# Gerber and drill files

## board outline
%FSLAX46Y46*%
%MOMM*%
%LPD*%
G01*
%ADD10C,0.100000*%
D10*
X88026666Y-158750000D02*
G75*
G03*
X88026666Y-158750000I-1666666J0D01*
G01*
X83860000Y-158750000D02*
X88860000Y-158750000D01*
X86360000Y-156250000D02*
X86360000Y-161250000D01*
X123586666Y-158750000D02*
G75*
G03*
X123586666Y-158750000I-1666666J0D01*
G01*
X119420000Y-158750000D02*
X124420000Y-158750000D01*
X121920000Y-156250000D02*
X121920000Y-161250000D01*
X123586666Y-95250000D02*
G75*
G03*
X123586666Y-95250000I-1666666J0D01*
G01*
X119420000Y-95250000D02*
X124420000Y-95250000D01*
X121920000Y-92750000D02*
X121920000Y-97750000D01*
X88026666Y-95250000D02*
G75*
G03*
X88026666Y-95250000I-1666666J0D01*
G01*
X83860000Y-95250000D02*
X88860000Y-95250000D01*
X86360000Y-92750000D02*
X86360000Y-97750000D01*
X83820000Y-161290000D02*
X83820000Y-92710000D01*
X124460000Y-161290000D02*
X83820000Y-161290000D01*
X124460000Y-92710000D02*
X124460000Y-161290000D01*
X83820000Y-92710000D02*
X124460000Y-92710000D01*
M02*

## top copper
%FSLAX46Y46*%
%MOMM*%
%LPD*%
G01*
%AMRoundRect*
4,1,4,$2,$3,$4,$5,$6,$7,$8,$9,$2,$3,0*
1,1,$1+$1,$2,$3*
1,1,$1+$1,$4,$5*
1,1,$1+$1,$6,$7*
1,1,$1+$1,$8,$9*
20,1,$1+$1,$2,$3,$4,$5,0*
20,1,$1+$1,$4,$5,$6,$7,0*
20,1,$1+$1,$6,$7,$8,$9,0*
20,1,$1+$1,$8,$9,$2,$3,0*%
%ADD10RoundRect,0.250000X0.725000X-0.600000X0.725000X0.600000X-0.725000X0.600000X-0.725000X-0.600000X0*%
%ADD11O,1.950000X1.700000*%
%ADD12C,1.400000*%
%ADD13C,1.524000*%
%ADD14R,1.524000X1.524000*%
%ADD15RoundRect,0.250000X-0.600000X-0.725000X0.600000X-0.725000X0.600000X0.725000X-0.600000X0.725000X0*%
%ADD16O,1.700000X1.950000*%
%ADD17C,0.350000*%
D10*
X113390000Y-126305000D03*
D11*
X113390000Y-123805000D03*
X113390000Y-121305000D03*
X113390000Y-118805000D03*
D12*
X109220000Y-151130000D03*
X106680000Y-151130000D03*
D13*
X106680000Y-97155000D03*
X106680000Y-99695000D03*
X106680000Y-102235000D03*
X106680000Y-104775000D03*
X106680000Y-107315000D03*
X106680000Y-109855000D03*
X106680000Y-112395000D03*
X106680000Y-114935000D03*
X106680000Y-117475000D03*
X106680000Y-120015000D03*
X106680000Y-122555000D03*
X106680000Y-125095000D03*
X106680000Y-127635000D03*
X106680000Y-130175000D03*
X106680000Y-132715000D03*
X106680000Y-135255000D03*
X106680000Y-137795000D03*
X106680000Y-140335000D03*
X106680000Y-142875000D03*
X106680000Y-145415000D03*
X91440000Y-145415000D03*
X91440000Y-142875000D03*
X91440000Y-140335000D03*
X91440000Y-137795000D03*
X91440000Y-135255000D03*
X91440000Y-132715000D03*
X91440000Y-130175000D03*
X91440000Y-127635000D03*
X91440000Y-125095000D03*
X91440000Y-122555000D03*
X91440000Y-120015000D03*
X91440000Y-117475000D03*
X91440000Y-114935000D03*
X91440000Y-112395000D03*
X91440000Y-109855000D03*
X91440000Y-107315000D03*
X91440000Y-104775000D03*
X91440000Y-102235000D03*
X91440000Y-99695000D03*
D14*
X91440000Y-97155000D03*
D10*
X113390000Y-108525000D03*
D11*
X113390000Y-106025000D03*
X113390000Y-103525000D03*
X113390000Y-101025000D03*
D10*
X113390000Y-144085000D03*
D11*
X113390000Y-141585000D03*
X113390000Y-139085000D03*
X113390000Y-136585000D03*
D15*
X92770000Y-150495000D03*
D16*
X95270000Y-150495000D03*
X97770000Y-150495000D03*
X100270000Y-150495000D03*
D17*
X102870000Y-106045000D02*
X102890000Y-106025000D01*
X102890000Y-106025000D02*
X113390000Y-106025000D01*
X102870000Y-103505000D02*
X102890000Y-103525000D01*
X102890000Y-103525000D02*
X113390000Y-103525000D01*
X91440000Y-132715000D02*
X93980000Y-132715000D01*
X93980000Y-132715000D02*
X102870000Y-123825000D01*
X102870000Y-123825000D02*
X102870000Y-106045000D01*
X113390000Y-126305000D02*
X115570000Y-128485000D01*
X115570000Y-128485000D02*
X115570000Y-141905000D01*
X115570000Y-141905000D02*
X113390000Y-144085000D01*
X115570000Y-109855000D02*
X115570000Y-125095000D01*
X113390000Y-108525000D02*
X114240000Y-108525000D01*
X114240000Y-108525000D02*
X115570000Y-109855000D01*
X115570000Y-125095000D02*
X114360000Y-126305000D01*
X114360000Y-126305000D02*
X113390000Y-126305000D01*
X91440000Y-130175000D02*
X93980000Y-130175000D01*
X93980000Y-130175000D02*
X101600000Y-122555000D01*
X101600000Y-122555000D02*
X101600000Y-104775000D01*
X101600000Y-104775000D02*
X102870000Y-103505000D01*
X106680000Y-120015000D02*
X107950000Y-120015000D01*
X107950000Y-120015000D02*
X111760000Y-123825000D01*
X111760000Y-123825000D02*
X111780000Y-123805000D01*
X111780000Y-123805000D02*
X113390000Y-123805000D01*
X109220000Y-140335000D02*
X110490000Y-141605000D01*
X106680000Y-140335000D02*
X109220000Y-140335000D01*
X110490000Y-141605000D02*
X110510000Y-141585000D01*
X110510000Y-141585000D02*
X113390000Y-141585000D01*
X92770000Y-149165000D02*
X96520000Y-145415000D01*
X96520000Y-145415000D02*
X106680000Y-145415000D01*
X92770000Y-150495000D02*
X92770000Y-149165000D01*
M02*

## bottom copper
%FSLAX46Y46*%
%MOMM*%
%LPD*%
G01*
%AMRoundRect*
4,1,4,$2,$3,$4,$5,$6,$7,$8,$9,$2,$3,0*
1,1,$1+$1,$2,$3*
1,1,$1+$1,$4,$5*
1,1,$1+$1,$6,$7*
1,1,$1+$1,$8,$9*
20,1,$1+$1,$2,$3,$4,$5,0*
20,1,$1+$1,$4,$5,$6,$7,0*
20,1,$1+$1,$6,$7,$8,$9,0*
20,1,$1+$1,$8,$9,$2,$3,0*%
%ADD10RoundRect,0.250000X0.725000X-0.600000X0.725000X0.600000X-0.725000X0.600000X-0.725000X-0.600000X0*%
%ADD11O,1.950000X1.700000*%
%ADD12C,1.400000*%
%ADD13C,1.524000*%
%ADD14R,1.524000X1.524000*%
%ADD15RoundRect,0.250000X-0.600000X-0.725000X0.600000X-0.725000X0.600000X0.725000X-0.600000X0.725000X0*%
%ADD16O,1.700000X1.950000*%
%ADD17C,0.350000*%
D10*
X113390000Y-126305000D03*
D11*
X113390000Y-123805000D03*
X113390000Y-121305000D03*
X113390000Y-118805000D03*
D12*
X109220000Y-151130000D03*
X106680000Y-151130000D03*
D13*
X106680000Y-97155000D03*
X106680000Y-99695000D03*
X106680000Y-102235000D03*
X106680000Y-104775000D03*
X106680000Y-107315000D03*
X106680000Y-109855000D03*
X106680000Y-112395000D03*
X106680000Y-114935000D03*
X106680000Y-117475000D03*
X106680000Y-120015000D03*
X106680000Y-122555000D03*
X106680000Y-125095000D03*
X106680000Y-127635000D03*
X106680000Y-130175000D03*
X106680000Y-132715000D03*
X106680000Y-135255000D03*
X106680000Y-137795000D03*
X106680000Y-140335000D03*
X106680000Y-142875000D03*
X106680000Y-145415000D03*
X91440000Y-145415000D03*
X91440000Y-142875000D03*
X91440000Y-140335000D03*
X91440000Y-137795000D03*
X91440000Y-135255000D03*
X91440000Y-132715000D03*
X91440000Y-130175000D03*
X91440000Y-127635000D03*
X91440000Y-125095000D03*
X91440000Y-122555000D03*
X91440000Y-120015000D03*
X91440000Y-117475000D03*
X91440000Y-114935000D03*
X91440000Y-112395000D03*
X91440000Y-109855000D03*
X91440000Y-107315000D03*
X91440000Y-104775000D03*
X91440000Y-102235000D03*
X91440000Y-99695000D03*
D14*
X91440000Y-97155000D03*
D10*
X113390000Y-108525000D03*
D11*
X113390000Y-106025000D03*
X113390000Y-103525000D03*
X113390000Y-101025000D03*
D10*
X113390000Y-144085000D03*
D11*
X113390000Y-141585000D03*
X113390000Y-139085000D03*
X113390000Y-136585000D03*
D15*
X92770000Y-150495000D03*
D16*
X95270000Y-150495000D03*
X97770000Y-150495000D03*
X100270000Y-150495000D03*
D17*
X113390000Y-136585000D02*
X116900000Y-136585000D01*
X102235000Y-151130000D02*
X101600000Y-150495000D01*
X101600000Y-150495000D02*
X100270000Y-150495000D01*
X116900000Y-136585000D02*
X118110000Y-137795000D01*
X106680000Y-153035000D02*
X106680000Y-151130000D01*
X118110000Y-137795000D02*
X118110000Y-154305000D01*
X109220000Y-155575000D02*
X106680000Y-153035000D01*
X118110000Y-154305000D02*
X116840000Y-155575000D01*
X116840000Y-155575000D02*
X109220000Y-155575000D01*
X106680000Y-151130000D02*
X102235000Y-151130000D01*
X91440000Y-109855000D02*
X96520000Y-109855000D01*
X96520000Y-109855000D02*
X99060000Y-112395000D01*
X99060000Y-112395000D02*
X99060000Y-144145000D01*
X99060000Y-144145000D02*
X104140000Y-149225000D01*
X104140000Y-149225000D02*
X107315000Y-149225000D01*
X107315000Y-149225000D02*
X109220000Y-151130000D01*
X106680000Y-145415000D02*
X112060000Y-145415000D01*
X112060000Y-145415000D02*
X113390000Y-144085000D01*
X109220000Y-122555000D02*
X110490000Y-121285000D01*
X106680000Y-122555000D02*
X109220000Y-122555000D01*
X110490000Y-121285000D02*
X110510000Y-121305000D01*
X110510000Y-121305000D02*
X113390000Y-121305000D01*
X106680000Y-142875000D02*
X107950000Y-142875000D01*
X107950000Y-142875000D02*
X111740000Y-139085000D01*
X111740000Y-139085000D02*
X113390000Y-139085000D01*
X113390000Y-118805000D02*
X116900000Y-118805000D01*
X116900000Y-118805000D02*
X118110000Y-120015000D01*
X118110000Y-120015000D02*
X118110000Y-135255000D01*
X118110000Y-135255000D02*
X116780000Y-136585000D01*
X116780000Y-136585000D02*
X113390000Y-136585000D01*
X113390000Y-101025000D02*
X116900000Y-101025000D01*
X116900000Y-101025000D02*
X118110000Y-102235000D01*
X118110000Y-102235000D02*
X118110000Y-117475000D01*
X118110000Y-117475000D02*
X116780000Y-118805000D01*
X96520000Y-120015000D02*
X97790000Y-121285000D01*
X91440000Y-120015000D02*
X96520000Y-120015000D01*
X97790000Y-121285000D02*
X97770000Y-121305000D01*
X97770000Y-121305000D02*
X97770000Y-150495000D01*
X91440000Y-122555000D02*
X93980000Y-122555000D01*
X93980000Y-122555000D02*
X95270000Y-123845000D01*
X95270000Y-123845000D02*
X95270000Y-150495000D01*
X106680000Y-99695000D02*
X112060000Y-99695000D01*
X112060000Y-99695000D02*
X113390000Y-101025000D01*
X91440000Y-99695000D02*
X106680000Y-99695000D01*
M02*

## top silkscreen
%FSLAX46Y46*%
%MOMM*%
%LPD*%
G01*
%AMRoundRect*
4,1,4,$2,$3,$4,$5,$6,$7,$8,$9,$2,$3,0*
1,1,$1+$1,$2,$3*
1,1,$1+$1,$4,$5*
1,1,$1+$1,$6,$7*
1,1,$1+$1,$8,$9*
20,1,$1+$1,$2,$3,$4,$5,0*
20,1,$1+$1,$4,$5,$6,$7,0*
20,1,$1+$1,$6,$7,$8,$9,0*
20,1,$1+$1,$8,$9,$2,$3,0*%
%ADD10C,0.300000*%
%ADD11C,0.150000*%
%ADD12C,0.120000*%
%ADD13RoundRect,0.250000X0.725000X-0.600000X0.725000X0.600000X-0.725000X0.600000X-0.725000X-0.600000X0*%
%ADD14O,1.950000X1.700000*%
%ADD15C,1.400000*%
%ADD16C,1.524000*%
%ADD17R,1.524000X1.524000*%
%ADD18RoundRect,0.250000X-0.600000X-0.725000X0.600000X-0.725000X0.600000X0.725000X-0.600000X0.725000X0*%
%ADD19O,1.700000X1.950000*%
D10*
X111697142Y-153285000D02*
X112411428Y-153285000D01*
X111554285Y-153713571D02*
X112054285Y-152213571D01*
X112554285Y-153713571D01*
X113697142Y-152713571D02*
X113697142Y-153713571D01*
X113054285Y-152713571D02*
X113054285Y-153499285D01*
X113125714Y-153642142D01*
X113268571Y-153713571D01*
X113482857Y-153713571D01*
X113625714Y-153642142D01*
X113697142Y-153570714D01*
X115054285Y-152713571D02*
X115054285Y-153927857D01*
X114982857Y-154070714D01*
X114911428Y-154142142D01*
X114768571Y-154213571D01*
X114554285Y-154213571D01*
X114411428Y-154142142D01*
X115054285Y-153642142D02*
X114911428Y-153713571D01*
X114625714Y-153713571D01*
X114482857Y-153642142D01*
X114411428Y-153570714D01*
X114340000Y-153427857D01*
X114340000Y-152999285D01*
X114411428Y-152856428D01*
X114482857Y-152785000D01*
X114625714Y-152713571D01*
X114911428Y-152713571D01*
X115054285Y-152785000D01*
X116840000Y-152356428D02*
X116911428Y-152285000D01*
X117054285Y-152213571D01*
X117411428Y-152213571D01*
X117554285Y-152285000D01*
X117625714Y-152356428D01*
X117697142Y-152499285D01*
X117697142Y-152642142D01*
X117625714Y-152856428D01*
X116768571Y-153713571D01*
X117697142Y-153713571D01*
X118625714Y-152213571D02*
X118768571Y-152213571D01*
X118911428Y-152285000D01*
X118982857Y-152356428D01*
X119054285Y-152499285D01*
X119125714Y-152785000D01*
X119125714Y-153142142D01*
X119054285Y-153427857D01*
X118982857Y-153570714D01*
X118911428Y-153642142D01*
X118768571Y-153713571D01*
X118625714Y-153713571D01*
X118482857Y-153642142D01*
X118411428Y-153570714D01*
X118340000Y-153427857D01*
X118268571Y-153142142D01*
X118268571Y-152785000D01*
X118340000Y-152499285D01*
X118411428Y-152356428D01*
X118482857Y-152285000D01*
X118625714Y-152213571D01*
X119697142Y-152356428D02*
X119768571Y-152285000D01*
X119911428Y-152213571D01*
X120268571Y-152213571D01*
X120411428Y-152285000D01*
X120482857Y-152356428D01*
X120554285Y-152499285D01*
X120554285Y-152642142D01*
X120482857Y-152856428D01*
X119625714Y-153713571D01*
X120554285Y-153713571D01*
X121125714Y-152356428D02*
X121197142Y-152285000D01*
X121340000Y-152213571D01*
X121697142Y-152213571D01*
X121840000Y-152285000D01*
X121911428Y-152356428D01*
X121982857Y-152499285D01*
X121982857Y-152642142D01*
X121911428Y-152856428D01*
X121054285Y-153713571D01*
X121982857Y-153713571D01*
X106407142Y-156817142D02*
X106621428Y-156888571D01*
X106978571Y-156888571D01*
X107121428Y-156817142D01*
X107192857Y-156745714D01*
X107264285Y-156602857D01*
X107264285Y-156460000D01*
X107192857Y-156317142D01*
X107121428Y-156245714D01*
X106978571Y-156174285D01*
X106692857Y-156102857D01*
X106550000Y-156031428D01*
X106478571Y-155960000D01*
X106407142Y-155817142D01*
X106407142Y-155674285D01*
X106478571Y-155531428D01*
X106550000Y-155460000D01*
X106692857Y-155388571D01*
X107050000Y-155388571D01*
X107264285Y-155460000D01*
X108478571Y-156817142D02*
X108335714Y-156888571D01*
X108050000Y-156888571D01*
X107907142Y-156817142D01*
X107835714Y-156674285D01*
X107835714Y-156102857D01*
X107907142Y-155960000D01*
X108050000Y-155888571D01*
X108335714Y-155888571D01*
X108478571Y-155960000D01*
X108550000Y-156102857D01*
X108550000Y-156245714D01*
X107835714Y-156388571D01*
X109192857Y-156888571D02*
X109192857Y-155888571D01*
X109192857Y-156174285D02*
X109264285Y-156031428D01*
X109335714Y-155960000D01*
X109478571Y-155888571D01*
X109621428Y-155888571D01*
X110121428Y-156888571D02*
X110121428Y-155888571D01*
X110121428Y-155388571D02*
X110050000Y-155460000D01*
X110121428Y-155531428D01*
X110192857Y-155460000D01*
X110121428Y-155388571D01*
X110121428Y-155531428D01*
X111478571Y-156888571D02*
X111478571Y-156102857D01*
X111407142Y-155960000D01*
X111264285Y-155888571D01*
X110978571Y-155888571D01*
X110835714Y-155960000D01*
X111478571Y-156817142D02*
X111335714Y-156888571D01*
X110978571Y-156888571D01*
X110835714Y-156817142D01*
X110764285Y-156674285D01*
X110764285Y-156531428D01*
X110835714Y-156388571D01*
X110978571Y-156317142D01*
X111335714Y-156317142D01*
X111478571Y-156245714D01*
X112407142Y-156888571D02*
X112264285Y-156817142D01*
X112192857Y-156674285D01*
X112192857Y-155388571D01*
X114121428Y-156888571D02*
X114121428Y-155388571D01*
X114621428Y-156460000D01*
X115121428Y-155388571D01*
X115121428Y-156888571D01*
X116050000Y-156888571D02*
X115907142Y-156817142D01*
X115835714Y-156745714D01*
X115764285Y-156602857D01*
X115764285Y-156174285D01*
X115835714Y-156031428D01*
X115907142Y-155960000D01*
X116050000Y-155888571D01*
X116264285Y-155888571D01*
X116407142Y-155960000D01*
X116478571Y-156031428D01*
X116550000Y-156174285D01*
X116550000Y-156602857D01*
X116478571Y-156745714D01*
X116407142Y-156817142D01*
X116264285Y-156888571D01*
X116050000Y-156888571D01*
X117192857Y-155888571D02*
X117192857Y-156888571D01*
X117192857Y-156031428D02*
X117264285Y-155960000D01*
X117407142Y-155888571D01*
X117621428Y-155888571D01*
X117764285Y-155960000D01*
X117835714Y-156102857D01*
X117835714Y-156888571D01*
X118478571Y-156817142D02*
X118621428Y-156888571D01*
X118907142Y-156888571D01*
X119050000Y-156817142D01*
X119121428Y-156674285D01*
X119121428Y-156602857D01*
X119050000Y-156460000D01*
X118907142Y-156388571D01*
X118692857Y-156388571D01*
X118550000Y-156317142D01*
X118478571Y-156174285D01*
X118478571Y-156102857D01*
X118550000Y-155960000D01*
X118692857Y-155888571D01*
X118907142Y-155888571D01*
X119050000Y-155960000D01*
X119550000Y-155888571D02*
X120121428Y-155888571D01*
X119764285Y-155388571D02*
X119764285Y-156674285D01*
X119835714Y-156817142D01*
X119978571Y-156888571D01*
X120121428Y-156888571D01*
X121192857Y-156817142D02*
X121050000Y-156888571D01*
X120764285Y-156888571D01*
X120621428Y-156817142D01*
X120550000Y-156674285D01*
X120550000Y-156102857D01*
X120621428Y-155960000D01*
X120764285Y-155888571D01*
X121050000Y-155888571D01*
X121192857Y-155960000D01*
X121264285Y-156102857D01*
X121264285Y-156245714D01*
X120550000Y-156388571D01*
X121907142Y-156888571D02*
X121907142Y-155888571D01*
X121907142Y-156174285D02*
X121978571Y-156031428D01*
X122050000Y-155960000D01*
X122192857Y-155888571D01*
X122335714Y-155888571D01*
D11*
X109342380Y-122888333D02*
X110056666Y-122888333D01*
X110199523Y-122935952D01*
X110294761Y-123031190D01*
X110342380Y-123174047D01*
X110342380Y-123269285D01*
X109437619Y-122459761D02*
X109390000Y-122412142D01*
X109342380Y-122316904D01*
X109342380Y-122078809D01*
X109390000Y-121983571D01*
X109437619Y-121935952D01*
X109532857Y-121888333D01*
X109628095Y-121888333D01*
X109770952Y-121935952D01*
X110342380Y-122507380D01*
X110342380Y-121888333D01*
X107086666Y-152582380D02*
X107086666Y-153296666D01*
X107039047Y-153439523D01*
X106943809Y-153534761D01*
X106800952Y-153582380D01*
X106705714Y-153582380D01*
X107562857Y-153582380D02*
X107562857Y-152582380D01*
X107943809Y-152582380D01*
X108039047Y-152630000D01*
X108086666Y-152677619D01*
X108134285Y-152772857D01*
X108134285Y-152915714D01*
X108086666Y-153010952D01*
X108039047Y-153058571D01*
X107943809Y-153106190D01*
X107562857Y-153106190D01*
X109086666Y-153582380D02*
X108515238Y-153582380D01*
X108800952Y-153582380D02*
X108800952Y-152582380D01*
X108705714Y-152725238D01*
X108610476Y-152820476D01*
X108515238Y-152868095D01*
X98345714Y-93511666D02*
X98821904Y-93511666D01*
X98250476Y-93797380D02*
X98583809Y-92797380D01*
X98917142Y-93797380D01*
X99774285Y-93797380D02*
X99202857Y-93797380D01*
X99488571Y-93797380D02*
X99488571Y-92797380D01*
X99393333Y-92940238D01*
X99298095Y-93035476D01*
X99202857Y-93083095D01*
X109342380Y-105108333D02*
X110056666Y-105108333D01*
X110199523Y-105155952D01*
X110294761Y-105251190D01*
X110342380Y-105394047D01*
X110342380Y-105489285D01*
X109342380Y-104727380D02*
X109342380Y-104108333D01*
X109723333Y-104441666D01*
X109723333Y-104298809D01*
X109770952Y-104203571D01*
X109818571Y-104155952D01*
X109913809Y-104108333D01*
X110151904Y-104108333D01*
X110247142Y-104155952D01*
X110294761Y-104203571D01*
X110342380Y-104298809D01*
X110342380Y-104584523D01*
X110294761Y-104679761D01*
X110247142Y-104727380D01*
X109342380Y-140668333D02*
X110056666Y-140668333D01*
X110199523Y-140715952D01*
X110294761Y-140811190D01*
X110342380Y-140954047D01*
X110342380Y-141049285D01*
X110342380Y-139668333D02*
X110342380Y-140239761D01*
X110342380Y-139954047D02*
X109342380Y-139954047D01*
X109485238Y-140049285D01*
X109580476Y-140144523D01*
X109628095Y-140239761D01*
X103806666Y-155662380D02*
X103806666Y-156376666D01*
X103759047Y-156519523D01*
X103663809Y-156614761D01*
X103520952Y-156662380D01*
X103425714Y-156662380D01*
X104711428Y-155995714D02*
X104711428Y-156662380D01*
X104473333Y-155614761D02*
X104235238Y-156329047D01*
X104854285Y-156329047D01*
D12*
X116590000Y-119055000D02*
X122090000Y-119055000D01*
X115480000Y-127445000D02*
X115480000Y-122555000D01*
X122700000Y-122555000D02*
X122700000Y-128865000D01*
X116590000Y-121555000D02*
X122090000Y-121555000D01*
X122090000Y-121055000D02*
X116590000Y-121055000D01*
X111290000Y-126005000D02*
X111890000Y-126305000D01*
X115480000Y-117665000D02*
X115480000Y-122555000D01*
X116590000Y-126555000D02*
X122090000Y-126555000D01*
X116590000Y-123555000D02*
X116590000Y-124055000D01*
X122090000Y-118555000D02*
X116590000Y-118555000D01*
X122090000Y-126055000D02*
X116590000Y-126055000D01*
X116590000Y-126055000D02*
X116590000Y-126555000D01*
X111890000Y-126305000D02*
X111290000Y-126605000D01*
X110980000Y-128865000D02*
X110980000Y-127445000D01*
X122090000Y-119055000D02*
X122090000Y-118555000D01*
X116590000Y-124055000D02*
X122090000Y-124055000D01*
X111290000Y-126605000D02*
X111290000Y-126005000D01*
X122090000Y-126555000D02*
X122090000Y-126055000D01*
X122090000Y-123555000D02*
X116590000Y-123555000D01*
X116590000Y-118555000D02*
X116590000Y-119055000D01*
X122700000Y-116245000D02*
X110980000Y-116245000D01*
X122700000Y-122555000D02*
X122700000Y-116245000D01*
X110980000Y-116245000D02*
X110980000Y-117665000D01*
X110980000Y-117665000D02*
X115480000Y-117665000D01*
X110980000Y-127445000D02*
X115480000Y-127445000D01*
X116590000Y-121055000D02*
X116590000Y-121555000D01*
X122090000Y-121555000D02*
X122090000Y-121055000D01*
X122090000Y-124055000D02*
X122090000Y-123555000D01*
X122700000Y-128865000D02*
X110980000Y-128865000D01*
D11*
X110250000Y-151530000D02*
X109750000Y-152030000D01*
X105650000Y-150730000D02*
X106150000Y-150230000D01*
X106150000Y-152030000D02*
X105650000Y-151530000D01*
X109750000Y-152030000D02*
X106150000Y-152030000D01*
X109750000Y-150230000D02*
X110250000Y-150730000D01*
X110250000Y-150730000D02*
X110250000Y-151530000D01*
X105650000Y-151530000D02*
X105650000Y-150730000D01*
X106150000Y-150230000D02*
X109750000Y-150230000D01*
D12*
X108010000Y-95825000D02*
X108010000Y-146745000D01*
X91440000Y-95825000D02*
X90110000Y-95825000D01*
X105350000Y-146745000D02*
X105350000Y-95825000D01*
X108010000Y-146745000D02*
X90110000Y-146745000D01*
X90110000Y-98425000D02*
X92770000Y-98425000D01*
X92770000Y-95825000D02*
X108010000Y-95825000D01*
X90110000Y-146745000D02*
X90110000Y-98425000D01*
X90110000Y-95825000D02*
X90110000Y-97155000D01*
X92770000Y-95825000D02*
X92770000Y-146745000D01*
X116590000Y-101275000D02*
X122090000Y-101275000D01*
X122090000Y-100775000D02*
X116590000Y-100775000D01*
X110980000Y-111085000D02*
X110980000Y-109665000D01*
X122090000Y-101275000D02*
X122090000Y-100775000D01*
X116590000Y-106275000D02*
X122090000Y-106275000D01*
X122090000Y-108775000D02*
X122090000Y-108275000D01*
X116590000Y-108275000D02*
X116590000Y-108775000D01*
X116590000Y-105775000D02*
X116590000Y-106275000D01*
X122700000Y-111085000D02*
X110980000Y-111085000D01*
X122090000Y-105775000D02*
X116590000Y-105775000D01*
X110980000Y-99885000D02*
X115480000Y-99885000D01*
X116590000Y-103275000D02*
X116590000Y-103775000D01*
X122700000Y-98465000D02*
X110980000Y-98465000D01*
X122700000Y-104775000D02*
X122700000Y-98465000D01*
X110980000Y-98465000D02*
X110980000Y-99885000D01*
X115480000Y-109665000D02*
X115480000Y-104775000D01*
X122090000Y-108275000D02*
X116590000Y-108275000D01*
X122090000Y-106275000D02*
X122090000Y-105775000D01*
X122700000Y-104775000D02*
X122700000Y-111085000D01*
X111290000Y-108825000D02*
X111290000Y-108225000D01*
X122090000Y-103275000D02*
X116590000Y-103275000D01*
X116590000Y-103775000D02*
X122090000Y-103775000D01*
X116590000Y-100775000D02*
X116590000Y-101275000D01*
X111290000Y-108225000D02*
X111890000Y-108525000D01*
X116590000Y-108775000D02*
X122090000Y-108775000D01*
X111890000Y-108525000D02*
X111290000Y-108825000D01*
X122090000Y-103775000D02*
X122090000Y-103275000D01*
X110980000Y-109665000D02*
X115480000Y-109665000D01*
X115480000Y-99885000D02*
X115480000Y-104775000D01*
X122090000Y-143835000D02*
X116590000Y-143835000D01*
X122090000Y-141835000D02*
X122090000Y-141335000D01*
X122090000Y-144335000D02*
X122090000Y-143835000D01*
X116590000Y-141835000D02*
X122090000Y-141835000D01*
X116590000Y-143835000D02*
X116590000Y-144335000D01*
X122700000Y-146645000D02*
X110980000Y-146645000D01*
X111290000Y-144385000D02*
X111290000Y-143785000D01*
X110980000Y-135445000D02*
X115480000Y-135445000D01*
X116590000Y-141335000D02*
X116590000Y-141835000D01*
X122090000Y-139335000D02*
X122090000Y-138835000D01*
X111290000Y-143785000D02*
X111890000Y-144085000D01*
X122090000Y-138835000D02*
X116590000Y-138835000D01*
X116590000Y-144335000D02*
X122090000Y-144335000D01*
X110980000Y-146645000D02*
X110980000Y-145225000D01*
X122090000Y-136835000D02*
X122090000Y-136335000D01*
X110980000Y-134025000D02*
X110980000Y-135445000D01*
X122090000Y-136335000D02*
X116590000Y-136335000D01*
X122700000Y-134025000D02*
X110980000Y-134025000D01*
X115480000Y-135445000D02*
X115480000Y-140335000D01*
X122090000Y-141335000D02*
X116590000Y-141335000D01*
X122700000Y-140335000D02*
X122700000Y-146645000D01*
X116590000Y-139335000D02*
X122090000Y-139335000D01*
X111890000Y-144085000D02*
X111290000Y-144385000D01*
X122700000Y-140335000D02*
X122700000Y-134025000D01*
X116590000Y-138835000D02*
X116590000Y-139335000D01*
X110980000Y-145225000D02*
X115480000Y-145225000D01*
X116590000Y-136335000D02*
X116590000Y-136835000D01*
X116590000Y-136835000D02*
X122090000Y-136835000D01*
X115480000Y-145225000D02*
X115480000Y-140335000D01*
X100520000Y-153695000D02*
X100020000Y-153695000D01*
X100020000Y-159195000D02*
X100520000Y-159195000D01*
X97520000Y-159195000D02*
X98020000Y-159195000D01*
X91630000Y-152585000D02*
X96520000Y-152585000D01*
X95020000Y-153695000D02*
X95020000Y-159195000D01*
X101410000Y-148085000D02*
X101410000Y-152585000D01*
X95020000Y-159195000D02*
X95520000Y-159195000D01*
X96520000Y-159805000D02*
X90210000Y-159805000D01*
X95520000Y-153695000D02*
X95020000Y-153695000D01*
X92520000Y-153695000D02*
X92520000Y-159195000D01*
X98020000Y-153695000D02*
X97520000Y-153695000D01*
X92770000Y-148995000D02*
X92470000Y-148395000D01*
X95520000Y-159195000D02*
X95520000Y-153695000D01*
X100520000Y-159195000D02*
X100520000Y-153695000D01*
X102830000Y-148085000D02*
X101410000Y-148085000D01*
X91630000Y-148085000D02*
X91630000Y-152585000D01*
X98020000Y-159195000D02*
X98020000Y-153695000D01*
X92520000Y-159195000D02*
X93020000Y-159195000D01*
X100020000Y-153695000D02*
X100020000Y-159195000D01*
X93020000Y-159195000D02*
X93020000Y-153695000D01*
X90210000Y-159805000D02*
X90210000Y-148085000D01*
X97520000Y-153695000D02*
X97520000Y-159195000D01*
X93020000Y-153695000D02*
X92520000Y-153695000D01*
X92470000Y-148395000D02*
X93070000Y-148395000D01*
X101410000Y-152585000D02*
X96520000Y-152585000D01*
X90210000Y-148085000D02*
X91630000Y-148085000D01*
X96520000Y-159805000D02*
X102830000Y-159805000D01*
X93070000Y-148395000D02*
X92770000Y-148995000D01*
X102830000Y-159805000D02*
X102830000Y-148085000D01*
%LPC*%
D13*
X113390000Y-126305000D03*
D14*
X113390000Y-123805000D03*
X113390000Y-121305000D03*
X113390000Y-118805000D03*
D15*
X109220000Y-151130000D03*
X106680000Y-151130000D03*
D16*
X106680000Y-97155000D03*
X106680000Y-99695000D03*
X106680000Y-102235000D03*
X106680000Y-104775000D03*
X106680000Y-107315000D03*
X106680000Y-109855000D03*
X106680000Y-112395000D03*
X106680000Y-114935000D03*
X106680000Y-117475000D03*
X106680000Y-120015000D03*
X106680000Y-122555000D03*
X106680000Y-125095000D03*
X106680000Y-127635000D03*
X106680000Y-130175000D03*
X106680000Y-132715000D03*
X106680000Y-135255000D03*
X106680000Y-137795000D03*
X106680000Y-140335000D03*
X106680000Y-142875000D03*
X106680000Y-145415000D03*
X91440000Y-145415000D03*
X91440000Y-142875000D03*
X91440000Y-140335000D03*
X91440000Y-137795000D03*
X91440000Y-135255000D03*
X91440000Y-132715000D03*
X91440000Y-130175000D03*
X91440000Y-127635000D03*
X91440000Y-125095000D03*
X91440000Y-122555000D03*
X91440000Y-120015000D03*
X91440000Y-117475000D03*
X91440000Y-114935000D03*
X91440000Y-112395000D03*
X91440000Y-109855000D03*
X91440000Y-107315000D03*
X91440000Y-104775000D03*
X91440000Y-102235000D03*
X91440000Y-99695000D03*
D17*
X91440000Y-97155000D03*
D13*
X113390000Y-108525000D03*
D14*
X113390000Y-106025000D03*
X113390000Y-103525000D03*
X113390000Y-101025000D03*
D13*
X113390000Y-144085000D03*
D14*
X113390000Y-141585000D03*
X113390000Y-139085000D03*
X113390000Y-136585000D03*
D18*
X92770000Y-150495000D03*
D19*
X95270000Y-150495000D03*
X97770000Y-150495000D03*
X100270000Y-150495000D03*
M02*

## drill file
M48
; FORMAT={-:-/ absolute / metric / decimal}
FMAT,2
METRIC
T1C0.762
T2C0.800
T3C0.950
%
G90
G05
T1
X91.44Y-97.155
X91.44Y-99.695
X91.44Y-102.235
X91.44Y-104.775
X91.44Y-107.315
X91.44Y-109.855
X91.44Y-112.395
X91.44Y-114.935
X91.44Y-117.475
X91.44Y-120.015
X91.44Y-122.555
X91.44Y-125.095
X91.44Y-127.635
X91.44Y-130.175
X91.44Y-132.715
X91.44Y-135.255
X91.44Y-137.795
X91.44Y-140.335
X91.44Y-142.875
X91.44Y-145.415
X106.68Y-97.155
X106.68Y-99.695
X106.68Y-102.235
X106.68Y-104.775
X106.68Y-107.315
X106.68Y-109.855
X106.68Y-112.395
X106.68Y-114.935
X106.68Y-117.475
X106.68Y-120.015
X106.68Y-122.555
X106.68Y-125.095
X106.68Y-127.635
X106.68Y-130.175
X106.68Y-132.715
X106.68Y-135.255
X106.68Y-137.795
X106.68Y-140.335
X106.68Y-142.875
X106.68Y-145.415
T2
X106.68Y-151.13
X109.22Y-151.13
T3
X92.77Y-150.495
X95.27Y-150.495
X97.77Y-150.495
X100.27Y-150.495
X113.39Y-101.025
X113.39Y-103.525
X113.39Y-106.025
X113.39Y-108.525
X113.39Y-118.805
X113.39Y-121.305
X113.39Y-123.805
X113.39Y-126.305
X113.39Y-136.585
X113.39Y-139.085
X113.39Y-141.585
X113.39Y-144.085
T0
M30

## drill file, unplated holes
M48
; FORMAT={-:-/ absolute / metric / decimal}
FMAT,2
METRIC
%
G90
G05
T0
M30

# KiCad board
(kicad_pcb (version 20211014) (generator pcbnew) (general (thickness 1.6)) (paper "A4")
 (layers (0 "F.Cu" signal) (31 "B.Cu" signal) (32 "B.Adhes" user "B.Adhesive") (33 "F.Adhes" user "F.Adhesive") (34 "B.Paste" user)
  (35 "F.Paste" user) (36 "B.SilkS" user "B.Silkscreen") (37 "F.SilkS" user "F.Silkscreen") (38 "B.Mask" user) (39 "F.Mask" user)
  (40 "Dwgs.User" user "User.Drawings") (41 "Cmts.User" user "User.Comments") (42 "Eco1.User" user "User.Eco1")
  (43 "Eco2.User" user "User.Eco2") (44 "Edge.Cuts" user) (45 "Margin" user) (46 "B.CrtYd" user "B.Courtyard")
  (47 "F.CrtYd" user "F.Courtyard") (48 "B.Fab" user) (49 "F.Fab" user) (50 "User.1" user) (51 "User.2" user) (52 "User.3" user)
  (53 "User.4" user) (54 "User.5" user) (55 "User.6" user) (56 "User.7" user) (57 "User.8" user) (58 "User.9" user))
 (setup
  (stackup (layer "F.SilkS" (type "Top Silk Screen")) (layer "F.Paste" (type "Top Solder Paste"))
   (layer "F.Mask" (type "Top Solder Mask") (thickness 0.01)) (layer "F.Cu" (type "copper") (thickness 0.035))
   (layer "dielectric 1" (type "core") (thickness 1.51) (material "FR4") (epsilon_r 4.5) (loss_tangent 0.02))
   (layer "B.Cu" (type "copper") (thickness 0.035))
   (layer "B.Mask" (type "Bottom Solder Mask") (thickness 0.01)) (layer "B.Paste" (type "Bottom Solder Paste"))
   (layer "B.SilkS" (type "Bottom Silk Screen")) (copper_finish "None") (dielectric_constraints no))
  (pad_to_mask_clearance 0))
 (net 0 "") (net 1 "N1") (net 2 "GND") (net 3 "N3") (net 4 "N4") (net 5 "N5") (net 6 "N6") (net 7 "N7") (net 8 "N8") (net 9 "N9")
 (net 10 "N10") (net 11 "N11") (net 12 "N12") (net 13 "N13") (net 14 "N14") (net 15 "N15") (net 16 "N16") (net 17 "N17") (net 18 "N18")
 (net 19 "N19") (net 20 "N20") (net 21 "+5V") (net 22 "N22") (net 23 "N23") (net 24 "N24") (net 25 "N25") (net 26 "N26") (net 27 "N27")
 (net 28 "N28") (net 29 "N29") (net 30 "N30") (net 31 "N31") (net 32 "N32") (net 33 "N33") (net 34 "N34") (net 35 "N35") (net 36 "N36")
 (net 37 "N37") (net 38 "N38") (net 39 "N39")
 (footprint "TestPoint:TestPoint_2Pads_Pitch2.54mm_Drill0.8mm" (layer "F.Cu") (at 109.22 151.13 180)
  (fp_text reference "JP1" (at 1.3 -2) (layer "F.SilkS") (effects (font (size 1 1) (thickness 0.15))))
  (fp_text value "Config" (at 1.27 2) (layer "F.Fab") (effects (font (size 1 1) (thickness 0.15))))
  (fp_line (start -1.03 0.4) (end -1.03 -0.4) (layer "F.SilkS") (width 0.15))
  (fp_line (start -0.53 0.9) (end -1.03 0.4) (layer "F.SilkS") (width 0.15))
  (fp_line (start -1.03 -0.4) (end -0.53 -0.9) (layer "F.SilkS") (width 0.15))
  (fp_line (start 3.07 -0.9) (end 3.57 -0.4) (layer "F.SilkS") (width 0.15))
  (fp_line (start 3.07 0.9) (end -0.53 0.9) (layer "F.SilkS") (width 0.15))
  (fp_line (start 3.57 -0.4) (end 3.57 0.4) (layer "F.SilkS") (width 0.15))
  (fp_line (start 3.57 0.4) (end 3.07 0.9) (layer "F.SilkS") (width 0.15))
  (fp_line (start -0.53 -0.9) (end 3.07 -0.9) (layer "F.SilkS") (width 0.15))
  (pad "1" thru_hole circle (at 0 0 180) (size 1.4 1.4) (drill 0.8) (layers *.Cu *.Mask) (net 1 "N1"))
  (pad "2" thru_hole circle (at 2.54 0 180) (size 1.4 1.4) (drill 0.8) (layers *.Cu *.Mask) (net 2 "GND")))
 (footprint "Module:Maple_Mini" (layer "F.Cu") (at 91.44 97.155)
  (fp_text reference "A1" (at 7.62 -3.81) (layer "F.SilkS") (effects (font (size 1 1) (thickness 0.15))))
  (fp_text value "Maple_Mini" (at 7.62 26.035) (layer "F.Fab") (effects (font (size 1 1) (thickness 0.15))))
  (fp_line (start 1.33 -1.33) (end 1.33 49.59) (layer "F.SilkS") (width 0.12))
  (fp_line (start -1.33 -1.33) (end -1.33 0) (layer "F.SilkS") (width 0.12))
  (fp_line (start -1.33 49.59) (end -1.33 1.27) (layer "F.SilkS") (width 0.12))
  (fp_line (start 1.33 -1.33) (end 16.57 -1.33) (layer "F.SilkS") (width 0.12))
  (fp_line (start -1.33 1.27) (end 1.33 1.27) (layer "F.SilkS") (width 0.12))
  (fp_line (start 16.57 49.59) (end -1.33 49.59) (layer "F.SilkS") (width 0.12))
  (fp_line (start 13.91 49.59) (end 13.91 -1.33) (layer "F.SilkS") (width 0.12))
  (fp_line (start 0 -1.33) (end -1.33 -1.33) (layer "F.SilkS") (width 0.12))
  (fp_line (start 16.57 -1.33) (end 16.57 49.59) (layer "F.SilkS") (width 0.12))
  (pad "1" thru_hole rect (at 0 0) (size 1.524 1.524) (drill 0.762) (layers *.Cu *.Mask) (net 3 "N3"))
  (pad "2" thru_hole circle (at 0 2.54) (size 1.524 1.524) (drill 0.762) (layers *.Cu *.Mask) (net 2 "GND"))
  (pad "3" thru_hole circle (at 0 5.08) (size 1.524 1.524) (drill 0.762) (layers *.Cu *.Mask) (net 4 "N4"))
  (pad "4" thru_hole circle (at 0 7.62) (size 1.524 1.524) (drill 0.762) (layers *.Cu *.Mask) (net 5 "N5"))
  (pad "5" thru_hole circle (at 0 10.16) (size 1.524 1.524) (drill 0.762) (layers *.Cu *.Mask) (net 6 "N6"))
  (pad "6" thru_hole circle (at 0 12.7) (size 1.524 1.524) (drill 0.762) (layers *.Cu *.Mask) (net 1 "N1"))
  (pad "7" thru_hole circle (at 0 15.24) (size 1.524 1.524) (drill 0.762) (layers *.Cu *.Mask) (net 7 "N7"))
  (pad "8" thru_hole circle (at 0 17.78) (size 1.524 1.524) (drill 0.762) (layers *.Cu *.Mask) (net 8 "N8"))
  (pad "9" thru_hole circle (at 0 20.32) (size 1.524 1.524) (drill 0.762) (layers *.Cu *.Mask) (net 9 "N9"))
  (pad "10" thru_hole circle (at 0 22.86) (size 1.524 1.524) (drill 0.762) (layers *.Cu *.Mask) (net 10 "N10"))
  (pad "11" thru_hole circle (at 0 25.4) (size 1.524 1.524) (drill 0.762) (layers *.Cu *.Mask) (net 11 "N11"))
  (pad "12" thru_hole circle (at 0 27.94) (size 1.524 1.524) (drill 0.762) (layers *.Cu *.Mask) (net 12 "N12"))
  (pad "13" thru_hole circle (at 0 30.48) (size 1.524 1.524) (drill 0.762) (layers *.Cu *.Mask) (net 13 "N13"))
  (pad "14" thru_hole circle (at 0 33.02) (size 1.524 1.524) (drill 0.762) (layers *.Cu *.Mask) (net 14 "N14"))
  (pad "15" thru_hole circle (at 0 35.56) (size 1.524 1.524) (drill 0.762) (layers *.Cu *.Mask) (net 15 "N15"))
  (pad "16" thru_hole circle (at 0 38.1) (size 1.524 1.524) (drill 0.762) (layers *.Cu *.Mask) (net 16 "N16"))
  (pad "17" thru_hole circle (at 0 40.64) (size 1.524 1.524) (drill 0.762) (layers *.Cu *.Mask) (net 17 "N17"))
  (pad "18" thru_hole circle (at 0 43.18) (size 1.524 1.524) (drill 0.762) (layers *.Cu *.Mask) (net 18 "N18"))
  (pad "19" thru_hole circle (at 0 45.72) (size 1.524 1.524) (drill 0.762) (layers *.Cu *.Mask) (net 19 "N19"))
  (pad "20" thru_hole circle (at 0 48.26) (size 1.524 1.524) (drill 0.762) (layers *.Cu *.Mask) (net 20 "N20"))
  (pad "21" thru_hole circle (at 15.24 48.26) (size 1.524 1.524) (drill 0.762) (layers *.Cu *.Mask) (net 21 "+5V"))
  (pad "22" thru_hole circle (at 15.24 45.72) (size 1.524 1.524) (drill 0.762) (layers *.Cu *.Mask) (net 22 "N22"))
  (pad "23" thru_hole circle (at 15.24 43.18) (size 1.524 1.524) (drill 0.762) (layers *.Cu *.Mask) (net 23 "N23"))
  (pad "24" thru_hole circle (at 15.24 40.64) (size 1.524 1.524) (drill 0.762) (layers *.Cu *.Mask) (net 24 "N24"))
  (pad "25" thru_hole circle (at 15.24 38.1) (size 1.524 1.524) (drill 0.762) (layers *.Cu *.Mask) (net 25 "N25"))
  (pad "26" thru_hole circle (at 15.24 35.56) (size 1.524 1.524) (drill 0.762) (layers *.Cu *.Mask) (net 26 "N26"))
  (pad "27" thru_hole circle (at 15.24 33.02) (size 1.524 1.524) (drill 0.762) (layers *.Cu *.Mask) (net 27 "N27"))
  (pad "28" thru_hole circle (at 15.24 30.48) (size 1.524 1.524) (drill 0.762) (layers *.Cu *.Mask) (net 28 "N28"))
  (pad "29" thru_hole circle (at 15.24 27.94) (size 1.524 1.524) (drill 0.762) (layers *.Cu *.Mask) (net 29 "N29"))
  (pad "30" thru_hole circle (at 15.24 25.4) (size 1.524 1.524) (drill 0.762) (layers *.Cu *.Mask) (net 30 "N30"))
  (pad "31" thru_hole circle (at 15.24 22.86) (size 1.524 1.524) (drill 0.762) (layers *.Cu *.Mask) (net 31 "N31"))
  (pad "32" thru_hole circle (at 15.24 20.32) (size 1.524 1.524) (drill 0.762) (layers *.Cu *.Mask) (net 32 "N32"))
  (pad "33" thru_hole circle (at 15.24 17.78) (size 1.524 1.524) (drill 0.762) (layers *.Cu *.Mask) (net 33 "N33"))
  (pad "34" thru_hole circle (at 15.24 15.24) (size 1.524 1.524) (drill 0.762) (layers *.Cu *.Mask) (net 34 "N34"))
  (pad "35" thru_hole circle (at 15.24 12.7) (size 1.524 1.524) (drill 0.762) (layers *.Cu *.Mask) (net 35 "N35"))
  (pad "36" thru_hole circle (at 15.24 10.16) (size 1.524 1.524) (drill 0.762) (layers *.Cu *.Mask) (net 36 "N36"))
  (pad "37" thru_hole circle (at 15.24 7.62) (size 1.524 1.524) (drill 0.762) (layers *.Cu *.Mask) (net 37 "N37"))
  (pad "38" thru_hole circle (at 15.24 5.08) (size 1.524 1.524) (drill 0.762) (layers *.Cu *.Mask) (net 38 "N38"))
  (pad "39" thru_hole circle (at 15.24 2.54) (size 1.524 1.524) (drill 0.762) (layers *.Cu *.Mask) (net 2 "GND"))
  (pad "40" thru_hole circle (at 15.24 0) (size 1.524 1.524) (drill 0.762) (layers *.Cu *.Mask) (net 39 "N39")))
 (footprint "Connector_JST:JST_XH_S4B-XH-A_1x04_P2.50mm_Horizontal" (layer "F.Cu") (at 113.39 126.305 90)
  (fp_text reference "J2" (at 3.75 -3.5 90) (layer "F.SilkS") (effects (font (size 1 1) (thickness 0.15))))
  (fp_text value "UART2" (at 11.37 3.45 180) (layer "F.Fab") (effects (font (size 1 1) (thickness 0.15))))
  (fp_line (start 7.25 3.2) (end 7.25 8.7) (layer "F.SilkS") (width 0.12))
  (fp_line (start -1.14 2.09) (end 3.75 2.09) (layer "F.SilkS") (width 0.12))
  (fp_line (start 3.75 9.31) (end -2.56 9.31) (layer "F.SilkS") (width 0.12))
  (fp_line (start 4.75 3.2) (end 4.75 8.7) (layer "F.SilkS") (width 0.12))
  (fp_line (start 5.25 8.7) (end 5.25 3.2) (layer "F.SilkS") (width 0.12))
  (fp_line (start 0.3 -2.1) (end 0 -1.5) (layer "F.SilkS") (width 0.12))
  (fp_line (start 8.64 2.09) (end 3.75 2.09) (layer "F.SilkS") (width 0.12))
  (fp_line (start -0.25 3.2) (end -0.25 8.7) (layer "F.SilkS") (width 0.12))
  (fp_line (start 2.75 3.2) (end 2.25 3.2) (layer "F.SilkS") (width 0.12))
  (fp_line (start 7.75 8.7) (end 7.75 3.2) (layer "F.SilkS") (width 0.12))
  (fp_line (start 0.25 8.7) (end 0.25 3.2) (layer "F.SilkS") (width 0.12))
  (fp_line (start 0.25 3.2) (end -0.25 3.2) (layer "F.SilkS") (width 0.12))
  (fp_line (start 0 -1.5) (end -0.3 -2.1) (layer "F.SilkS") (width 0.12))
  (fp_line (start -2.56 -2.41) (end -1.14 -2.41) (layer "F.SilkS") (width 0.12))
  (fp_line (start 7.25 8.7) (end 7.75 8.7) (layer "F.SilkS") (width 0.12))
  (fp_line (start 2.25 3.2) (end 2.25 8.7) (layer "F.SilkS") (width 0.12))
  (fp_line (start -0.3 -2.1) (end 0.3 -2.1) (layer "F.SilkS") (width 0.12))
  (fp_line (start -0.25 8.7) (end 0.25 8.7) (layer "F.SilkS") (width 0.12))
  (fp_line (start 2.75 8.7) (end 2.75 3.2) (layer "F.SilkS") (width 0.12))
  (fp_line (start 7.75 3.2) (end 7.25 3.2) (layer "F.SilkS") (width 0.12))
  (fp_line (start 10.06 9.31) (end 10.06 -2.41) (layer "F.SilkS") (width 0.12))
  (fp_line (start 3.75 9.31) (end 10.06 9.31) (layer "F.SilkS") (width 0.12))
  (fp_line (start 10.06 -2.41) (end 8.64 -2.41) (layer "F.SilkS") (width 0.12))
  (fp_line (start 8.64 -2.41) (end 8.64 2.09) (layer "F.SilkS") (width 0.12))
  (fp_line (start -1.14 -2.41) (end -1.14 2.09) (layer "F.SilkS") (width 0.12))
  (fp_line (start 5.25 3.2) (end 4.75 3.2) (layer "F.SilkS") (width 0.12))
  (fp_line (start 4.75 8.7) (end 5.25 8.7) (layer "F.SilkS") (width 0.12))
  (fp_line (start 2.25 8.7) (end 2.75 8.7) (layer "F.SilkS") (width 0.12))
  (fp_line (start -2.56 9.31) (end -2.56 -2.41) (layer "F.SilkS") (width 0.12))
  (pad "1" thru_hole roundrect (at 0 0 90) (size 1.7 1.95) (drill 0.95) (layers *.Cu *.Mask) (roundrect_rratio 0.1470588235) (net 21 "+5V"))
  (pad "2" thru_hole oval (at 2.5 0 90) (size 1.7 1.95) (drill 0.95) (layers *.Cu *.Mask) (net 31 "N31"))
  (pad "3" thru_hole oval (at 5 0 90) (size 1.7 1.95) (drill 0.95) (layers *.Cu *.Mask) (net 30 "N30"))
  (pad "4" thru_hole oval (at 7.5 0 90) (size 1.7 1.95) (drill 0.95) (layers *.Cu *.Mask) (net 2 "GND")))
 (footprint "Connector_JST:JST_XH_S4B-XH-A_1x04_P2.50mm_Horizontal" (layer "F.Cu") (at 113.39 108.525 90)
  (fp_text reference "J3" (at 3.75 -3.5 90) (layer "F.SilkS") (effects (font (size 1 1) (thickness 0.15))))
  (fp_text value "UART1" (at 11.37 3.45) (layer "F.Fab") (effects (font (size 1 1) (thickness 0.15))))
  (fp_line (start 7.25 3.2) (end 7.25 8.7) (layer "F.SilkS") (width 0.12))
  (fp_line (start 7.75 8.7) (end 7.75 3.2) (layer "F.SilkS") (width 0.12))
  (fp_line (start -2.56 -2.41) (end -1.14 -2.41) (layer "F.SilkS") (width 0.12))
  (fp_line (start 7.25 8.7) (end 7.75 8.7) (layer "F.SilkS") (width 0.12))
  (fp_line (start 2.25 3.2) (end 2.25 8.7) (layer "F.SilkS") (width 0.12))
  (fp_line (start -0.25 8.7) (end 0.25 8.7) (layer "F.SilkS") (width 0.12))
  (fp_line (start 0.25 3.2) (end -0.25 3.2) (layer "F.SilkS") (width 0.12))
  (fp_line (start 2.75 3.2) (end 2.25 3.2) (layer "F.SilkS") (width 0.12))
  (fp_line (start -2.56 9.31) (end -2.56 -2.41) (layer "F.SilkS") (width 0.12))
  (fp_line (start 2.75 8.7) (end 2.75 3.2) (layer "F.SilkS") (width 0.12))
  (fp_line (start 8.64 -2.41) (end 8.64 2.09) (layer "F.SilkS") (width 0.12))
  (fp_line (start 5.25 3.2) (end 4.75 3.2) (layer "F.SilkS") (width 0.12))
  (fp_line (start 10.06 9.31) (end 10.06 -2.41) (layer "F.SilkS") (width 0.12))
  (fp_line (start 3.75 9.31) (end 10.06 9.31) (layer "F.SilkS") (width 0.12))
  (fp_line (start 10.06 -2.41) (end 8.64 -2.41) (layer "F.SilkS") (width 0.12))
  (fp_line (start -1.14 2.09) (end 3.75 2.09) (layer "F.SilkS") (width 0.12))
  (fp_line (start 0.25 8.7) (end 0.25 3.2) (layer "F.SilkS") (width 0.12))
  (fp_line (start 2.25 8.7) (end 2.75 8.7) (layer "F.SilkS") (width 0.12))
  (fp_line (start 3.75 9.31) (end -2.56 9.31) (layer "F.SilkS") (width 0.12))
  (fp_line (start -0.3 -2.1) (end 0.3 -2.1) (layer "F.SilkS") (width 0.12))
  (fp_line (start 5.25 8.7) (end 5.25 3.2) (layer "F.SilkS") (width 0.12))
  (fp_line (start 4.75 3.2) (end 4.75 8.7) (layer "F.SilkS") (width 0.12))
  (fp_line (start 7.75 3.2) (end 7.25 3.2) (layer "F.SilkS") (width 0.12))
  (fp_line (start 0.3 -2.1) (end 0 -1.5) (layer "F.SilkS") (width 0.12))
  (fp_line (start -0.25 3.2) (end -0.25 8.7) (layer "F.SilkS") (width 0.12))
  (fp_line (start 0 -1.5) (end -0.3 -2.1) (layer "F.SilkS") (width 0.12))
  (fp_line (start 4.75 8.7) (end 5.25 8.7) (layer "F.SilkS") (width 0.12))
  (fp_line (start -1.14 -2.41) (end -1.14 2.09) (layer "F.SilkS") (width 0.12))
  (fp_line (start 8.64 2.09) (end 3.75 2.09) (layer "F.SilkS") (width 0.12))
  (pad "1" thru_hole roundrect (at 0 0 90) (size 1.7 1.95) (drill 0.95) (layers *.Cu *.Mask) (roundrect_rratio 0.1470588235) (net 21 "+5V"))
  (pad "2" thru_hole oval (at 2.5 0 90) (size 1.7 1.95) (drill 0.95) (layers *.Cu *.Mask) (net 15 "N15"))
  (pad "3" thru_hole oval (at 5 0 90) (size 1.7 1.95) (drill 0.95) (layers *.Cu *.Mask) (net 14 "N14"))
  (pad "4" thru_hole oval (at 7.5 0 90) (size 1.7 1.95) (drill 0.95) (layers *.Cu *.Mask) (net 2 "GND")))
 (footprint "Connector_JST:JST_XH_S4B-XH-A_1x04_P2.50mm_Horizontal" (layer "F.Cu") (at 113.39 144.085 90)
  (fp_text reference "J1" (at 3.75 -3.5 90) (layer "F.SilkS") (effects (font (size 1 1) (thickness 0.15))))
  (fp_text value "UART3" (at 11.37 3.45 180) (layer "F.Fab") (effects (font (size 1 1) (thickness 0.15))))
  (fp_line (start 0.25 8.7) (end 0.25 3.2) (layer "F.SilkS") (width 0.12))
  (fp_line (start 2.25 8.7) (end 2.75 8.7) (layer "F.SilkS") (width 0.12))
  (fp_line (start -0.25 8.7) (end 0.25 8.7) (layer "F.SilkS") (width 0.12))
  (fp_line (start 2.25 3.2) (end 2.25 8.7) (layer "F.SilkS") (width 0.12))
  (fp_line (start 0.25 3.2) (end -0.25 3.2) (layer "F.SilkS") (width 0.12))
  (fp_line (start -2.56 9.31) (end -2.56 -2.41) (layer "F.SilkS") (width 0.12))
  (fp_line (start -0.3 -2.1) (end 0.3 -2.1) (layer "F.SilkS") (width 0.12))
  (fp_line (start 8.64 -2.41) (end 8.64 2.09) (layer "F.SilkS") (width 0.12))
  (fp_line (start 2.75 3.2) (end 2.25 3.2) (layer "F.SilkS") (width 0.12))
  (fp_line (start 4.75 8.7) (end 5.25 8.7) (layer "F.SilkS") (width 0.12))
  (fp_line (start 0.3 -2.1) (end 0 -1.5) (layer "F.SilkS") (width 0.12))
  (fp_line (start 5.25 8.7) (end 5.25 3.2) (layer "F.SilkS") (width 0.12))
  (fp_line (start -0.25 3.2) (end -0.25 8.7) (layer "F.SilkS") (width 0.12))
  (fp_line (start -2.56 -2.41) (end -1.14 -2.41) (layer "F.SilkS") (width 0.12))
  (fp_line (start 7.25 8.7) (end 7.75 8.7) (layer "F.SilkS") (width 0.12))
  (fp_line (start 10.06 -2.41) (end 8.64 -2.41) (layer "F.SilkS") (width 0.12))
  (fp_line (start 7.75 8.7) (end 7.75 3.2) (layer "F.SilkS") (width 0.12))
  (fp_line (start 10.06 9.31) (end 10.06 -2.41) (layer "F.SilkS") (width 0.12))
  (fp_line (start 8.64 2.09) (end 3.75 2.09) (layer "F.SilkS") (width 0.12))
  (fp_line (start 2.75 8.7) (end 2.75 3.2) (layer "F.SilkS") (width 0.12))
  (fp_line (start 3.75 9.31) (end -2.56 9.31) (layer "F.SilkS") (width 0.12))
  (fp_line (start 4.75 3.2) (end 4.75 8.7) (layer "F.SilkS") (width 0.12))
  (fp_line (start 0 -1.5) (end -0.3 -2.1) (layer "F.SilkS") (width 0.12))
  (fp_line (start 3.75 9.31) (end 10.06 9.31) (layer "F.SilkS") (width 0.12))
  (fp_line (start 5.25 3.2) (end 4.75 3.2) (layer "F.SilkS") (width 0.12))
  (fp_line (start -1.14 -2.41) (end -1.14 2.09) (layer "F.SilkS") (width 0.12))
  (fp_line (start 7.75 3.2) (end 7.25 3.2) (layer "F.SilkS") (width 0.12))
  (fp_line (start 7.25 3.2) (end 7.25 8.7) (layer "F.SilkS") (width 0.12))
  (fp_line (start -1.14 2.09) (end 3.75 2.09) (layer "F.SilkS") (width 0.12))
  (pad "1" thru_hole roundrect (at 0 0 90) (size 1.7 1.95) (drill 0.95) (layers *.Cu *.Mask) (roundrect_rratio 0.1470588235) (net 21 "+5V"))
  (pad "2" thru_hole oval (at 2.5 0 90) (size 1.7 1.95) (drill 0.95) (layers *.Cu *.Mask) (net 23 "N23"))
  (pad "3" thru_hole oval (at 5 0 90) (size 1.7 1.95) (drill 0.95) (layers *.Cu *.Mask) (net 22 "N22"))
  (pad "4" thru_hole oval (at 7.5 0 90) (size 1.7 1.95) (drill 0.95) (layers *.Cu *.Mask) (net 2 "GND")))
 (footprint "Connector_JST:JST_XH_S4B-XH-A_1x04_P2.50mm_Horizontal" (layer "F.Cu") (at 92.77 150.495)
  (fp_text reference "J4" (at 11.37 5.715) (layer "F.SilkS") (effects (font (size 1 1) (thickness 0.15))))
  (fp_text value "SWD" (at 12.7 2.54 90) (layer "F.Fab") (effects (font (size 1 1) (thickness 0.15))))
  (fp_line (start 7.75 3.2) (end 7.25 3.2) (layer "F.SilkS") (width 0.12))
  (fp_line (start 7.25 8.7) (end 7.75 8.7) (layer "F.SilkS") (width 0.12))
  (fp_line (start 4.75 8.7) (end 5.25 8.7) (layer "F.SilkS") (width 0.12))
  (fp_line (start -1.14 2.09) (end 3.75 2.09) (layer "F.SilkS") (width 0.12))
  (fp_line (start 2.25 3.2) (end 2.25 8.7) (layer "F.SilkS") (width 0.12))
  (fp_line (start 8.64 -2.41) (end 8.64 2.09) (layer "F.SilkS") (width 0.12))
  (fp_line (start 2.25 8.7) (end 2.75 8.7) (layer "F.SilkS") (width 0.12))
  (fp_line (start 3.75 9.31) (end -2.56 9.31) (layer "F.SilkS") (width 0.12))
  (fp_line (start 2.75 3.2) (end 2.25 3.2) (layer "F.SilkS") (width 0.12))
  (fp_line (start -0.25 3.2) (end -0.25 8.7) (layer "F.SilkS") (width 0.12))
  (fp_line (start 5.25 3.2) (end 4.75 3.2) (layer "F.SilkS") (width 0.12))
  (fp_line (start 0 -1.5) (end -0.3 -2.1) (layer "F.SilkS") (width 0.12))
  (fp_line (start 2.75 8.7) (end 2.75 3.2) (layer "F.SilkS") (width 0.12))
  (fp_line (start 7.75 8.7) (end 7.75 3.2) (layer "F.SilkS") (width 0.12))
  (fp_line (start 10.06 -2.41) (end 8.64 -2.41) (layer "F.SilkS") (width 0.12))
  (fp_line (start -1.14 -2.41) (end -1.14 2.09) (layer "F.SilkS") (width 0.12))
  (fp_line (start 5.25 8.7) (end 5.25 3.2) (layer "F.SilkS") (width 0.12))
  (fp_line (start -0.25 8.7) (end 0.25 8.7) (layer "F.SilkS") (width 0.12))
  (fp_line (start 7.25 3.2) (end 7.25 8.7) (layer "F.SilkS") (width 0.12))
  (fp_line (start 0.25 8.7) (end 0.25 3.2) (layer "F.SilkS") (width 0.12))
  (fp_line (start -2.56 9.31) (end -2.56 -2.41) (layer "F.SilkS") (width 0.12))
  (fp_line (start 4.75 3.2) (end 4.75 8.7) (layer "F.SilkS") (width 0.12))
  (fp_line (start 0.25 3.2) (end -0.25 3.2) (layer "F.SilkS") (width 0.12))
  (fp_line (start -0.3 -2.1) (end 0.3 -2.1) (layer "F.SilkS") (width 0.12))
  (fp_line (start 8.64 2.09) (end 3.75 2.09) (layer "F.SilkS") (width 0.12))
  (fp_line (start -2.56 -2.41) (end -1.14 -2.41) (layer "F.SilkS") (width 0.12))
  (fp_line (start 3.75 9.31) (end 10.06 9.31) (layer "F.SilkS") (width 0.12))
  (fp_line (start 0.3 -2.1) (end 0 -1.5) (layer "F.SilkS") (width 0.12))
  (fp_line (start 10.06 9.31) (end 10.06 -2.41) (layer "F.SilkS") (width 0.12))
  (pad "1" thru_hole roundrect (at 0 0) (size 1.7 1.95) (drill 0.95) (layers *.Cu *.Mask) (roundrect_rratio 0.1470588235) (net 21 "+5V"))
  (pad "2" thru_hole oval (at 2.5 0) (size 1.7 1.95) (drill 0.95) (layers *.Cu *.Mask) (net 11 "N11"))
  (pad "3" thru_hole oval (at 5 0) (size 1.7 1.95) (drill 0.95) (layers *.Cu *.Mask) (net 10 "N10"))
  (pad "4" thru_hole oval (at 7.5 0) (size 1.7 1.95) (drill 0.95) (layers *.Cu *.Mask) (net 2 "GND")))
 (gr_line (start 124.46 92.71) (end 124.46 161.29) (layer "Edge.Cuts") (width 0.1))
 (gr_line (start 124.46 161.29) (end 83.82 161.29) (layer "Edge.Cuts") (width 0.1))
 (gr_line (start 83.82 92.71) (end 124.46 92.71) (layer "Edge.Cuts") (width 0.1))
 (gr_line (start 83.82 161.29) (end 83.82 92.71) (layer "Edge.Cuts") (width 0.1))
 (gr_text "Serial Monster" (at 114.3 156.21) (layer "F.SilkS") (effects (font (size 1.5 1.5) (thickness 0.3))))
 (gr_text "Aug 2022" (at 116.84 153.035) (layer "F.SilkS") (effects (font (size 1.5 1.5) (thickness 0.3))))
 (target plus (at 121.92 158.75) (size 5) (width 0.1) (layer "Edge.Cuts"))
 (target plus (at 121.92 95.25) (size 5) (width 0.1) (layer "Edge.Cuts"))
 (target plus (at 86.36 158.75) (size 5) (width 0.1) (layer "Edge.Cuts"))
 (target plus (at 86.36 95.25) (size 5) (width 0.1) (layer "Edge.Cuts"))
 (segment (start 106.68 151.13) (end 102.235 151.13) (width 0.35) (layer "B.Cu") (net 2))
 (segment (start 116.84 155.575) (end 109.22 155.575) (width 0.35) (layer "B.Cu") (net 2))
 (segment (start 116.9 101.025) (end 118.11 102.235) (width 0.35) (layer "B.Cu") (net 2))
 (segment (start 118.11 154.305) (end 116.84 155.575) (width 0.35) (layer "B.Cu") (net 2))
 (segment (start 101.6 150.495) (end 100.27 150.495) (width 0.35) (layer "B.Cu") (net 2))
 (segment (start 113.39 136.585) (end 116.9 136.585) (width 0.35) (layer "B.Cu") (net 2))
 (segment (start 106.68 99.695) (end 112.06 99.695) (width 0.35) (layer "B.Cu") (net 2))
 (segment (start 102.235 151.13) (end 101.6 150.495) (width 0.35) (layer "B.Cu") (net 2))
 (segment (start 106.68 153.035) (end 106.68 151.13) (width 0.35) (layer "B.Cu") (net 2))
 (segment (start 118.11 135.255) (end 116.78 136.585) (width 0.35) (layer "B.Cu") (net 2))
 (segment (start 113.39 101.025) (end 116.9 101.025) (width 0.35) (layer "B.Cu") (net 2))
 (segment (start 118.11 102.235) (end 118.11 117.475) (width 0.35) (layer "B.Cu") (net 2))
 (segment (start 116.9 136.585) (end 118.11 137.795) (width 0.35) (layer "B.Cu") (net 2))
 (segment (start 112.06 99.695) (end 113.39 101.025) (width 0.35) (layer "B.Cu") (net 2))
 (segment (start 118.11 137.795) (end 118.11 154.305) (width 0.35) (layer "B.Cu") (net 2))
 (segment (start 109.22 155.575) (end 106.68 153.035) (width 0.35) (layer "B.Cu") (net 2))
 (segment (start 116.9 118.805) (end 118.11 120.015) (width 0.35) (layer "B.Cu") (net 2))
 (segment (start 113.39 118.805) (end 116.9 118.805) (width 0.35) (layer "B.Cu") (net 2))
 (segment (start 118.11 117.475) (end 116.78 118.805) (width 0.35) (layer "B.Cu") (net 2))
 (segment (start 116.78 136.585) (end 113.39 136.585) (width 0.35) (layer "B.Cu") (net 2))
 (segment (start 118.11 120.015) (end 118.11 135.255) (width 0.35) (layer "B.Cu") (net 2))
 (segment (start 91.44 99.695) (end 106.68 99.695) (width 0.35) (layer "B.Cu") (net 2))
 (segment (start 99.06 144.145) (end 104.14 149.225) (width 0.35) (layer "B.Cu") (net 1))
 (segment (start 91.44 109.855) (end 96.52 109.855) (width 0.35) (layer "B.Cu") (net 1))
 (segment (start 99.06 112.395) (end 99.06 144.145) (width 0.35) (layer "B.Cu") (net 1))
 (segment (start 107.315 149.225) (end 109.22 151.13) (width 0.35) (layer "B.Cu") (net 1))
 (segment (start 104.14 149.225) (end 107.315 149.225) (width 0.35) (layer "B.Cu") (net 1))
 (segment (start 96.52 109.855) (end 99.06 112.395) (width 0.35) (layer "B.Cu") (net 1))
 (segment (start 102.87 103.505) (end 102.89 103.525) (width 0.35) (layer "F.Cu") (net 14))
 (segment (start 101.6 122.555) (end 101.6 104.775) (width 0.35) (layer "F.Cu") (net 14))
 (segment (start 102.89 103.525) (end 113.39 103.525) (width 0.35) (layer "F.Cu") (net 14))
 (segment (start 91.44 130.175) (end 93.98 130.175) (width 0.35) (layer "F.Cu") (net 14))
 (segment (start 93.98 130.175) (end 101.6 122.555) (width 0.35) (layer "F.Cu") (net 14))
 (segment (start 101.6 104.775) (end 102.87 103.505) (width 0.35) (layer "F.Cu") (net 14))
 (segment (start 91.44 132.715) (end 93.98 132.715) (width 0.35) (layer "F.Cu") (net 15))
 (segment (start 102.89 106.025) (end 113.39 106.025) (width 0.35) (layer "F.Cu") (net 15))
 (segment (start 102.87 106.045) (end 102.89 106.025) (width 0.35) (layer "F.Cu") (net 15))
 (segment (start 93.98 132.715) (end 102.87 123.825) (width 0.35) (layer "F.Cu") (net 15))
 (segment (start 102.87 123.825) (end 102.87 106.045) (width 0.35) (layer "F.Cu") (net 15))
 (segment (start 113.39 126.305) (end 115.57 128.485) (width 0.35) (layer "F.Cu") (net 21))
 (segment (start 92.77 149.165) (end 96.52 145.415) (width 0.35) (layer "F.Cu") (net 21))
 (segment (start 114.24 108.525) (end 115.57 109.855) (width 0.35) (layer "F.Cu") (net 21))
 (segment (start 92.77 150.495) (end 92.77 149.165) (width 0.35) (layer "F.Cu") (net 21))
 (segment (start 115.57 109.855) (end 115.57 125.095) (width 0.35) (layer "F.Cu") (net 21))
 (segment (start 114.36 126.305) (end 113.39 126.305) (width 0.35) (layer "F.Cu") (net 21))
 (segment (start 115.57 128.485) (end 115.57 141.905) (width 0.35) (layer "F.Cu") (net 21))
 (segment (start 115.57 141.905) (end 113.39 144.085) (width 0.35) (layer "F.Cu") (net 21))
 (segment (start 115.57 125.095) (end 114.36 126.305) (width 0.35) (layer "F.Cu") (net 21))
 (segment (start 113.39 108.525) (end 114.24 108.525) (width 0.35) (layer "F.Cu") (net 21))
 (segment (start 96.52 145.415) (end 106.68 145.415) (width 0.35) (layer "F.Cu") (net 21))
 (segment (start 112.06 145.415) (end 113.39 144.085) (width 0.35) (layer "B.Cu") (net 21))
 (segment (start 106.68 145.415) (end 112.06 145.415) (width 0.35) (layer "B.Cu") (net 21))
 (segment (start 106.68 142.875) (end 107.95 142.875) (width 0.35) (layer "B.Cu") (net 22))
 (segment (start 107.95 142.875) (end 111.74 139.085) (width 0.35) (layer "B.Cu") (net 22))
 (segment (start 111.74 139.085) (end 113.39 139.085) (width 0.35) (layer "B.Cu") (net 22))
 (segment (start 110.51 141.585) (end 113.39 141.585) (width 0.35) (layer "F.Cu") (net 23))
 (segment (start 106.68 140.335) (end 109.22 140.335) (width 0.35) (layer "F.Cu") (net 23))
 (segment (start 109.22 140.335) (end 110.49 141.605) (width 0.35) (layer "F.Cu") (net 23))
 (segment (start 110.49 141.605) (end 110.51 141.585) (width 0.35) (layer "F.Cu") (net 23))
 (segment (start 110.49 121.285) (end 110.51 121.305) (width 0.35) (layer "B.Cu") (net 30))
 (segment (start 109.22 122.555) (end 110.49 121.285) (width 0.35) (layer "B.Cu") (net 30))
 (segment (start 106.68 122.555) (end 109.22 122.555) (width 0.35) (layer "B.Cu") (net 30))
 (segment (start 110.51 121.305) (end 113.39 121.305) (width 0.35) (layer "B.Cu") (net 30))
 (segment (start 111.78 123.805) (end 113.39 123.805) (width 0.35) (layer "F.Cu") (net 31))
 (segment (start 111.76 123.825) (end 111.78 123.805) (width 0.35) (layer "F.Cu") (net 31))
 (segment (start 107.95 120.015) (end 111.76 123.825) (width 0.35) (layer "F.Cu") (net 31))
 (segment (start 106.68 120.015) (end 107.95 120.015) (width 0.35) (layer "F.Cu") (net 31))
 (segment (start 97.77 121.305) (end 97.77 150.495) (width 0.35) (layer "B.Cu") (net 10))
 (segment (start 96.52 120.015) (end 97.79 121.285) (width 0.35) (layer "B.Cu") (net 10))
 (segment (start 97.79 121.285) (end 97.77 121.305) (width 0.35) (layer "B.Cu") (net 10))
 (segment (start 91.44 120.015) (end 96.52 120.015) (width 0.35) (layer "B.Cu") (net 10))
 (segment (start 95.27 123.845) (end 95.27 150.495) (width 0.35) (layer "B.Cu") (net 11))
 (segment (start 91.44 122.555) (end 93.98 122.555) (width 0.35) (layer "B.Cu") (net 11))
 (segment (start 93.98 122.555) (end 95.27 123.845) (width 0.35) (layer "B.Cu") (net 11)))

